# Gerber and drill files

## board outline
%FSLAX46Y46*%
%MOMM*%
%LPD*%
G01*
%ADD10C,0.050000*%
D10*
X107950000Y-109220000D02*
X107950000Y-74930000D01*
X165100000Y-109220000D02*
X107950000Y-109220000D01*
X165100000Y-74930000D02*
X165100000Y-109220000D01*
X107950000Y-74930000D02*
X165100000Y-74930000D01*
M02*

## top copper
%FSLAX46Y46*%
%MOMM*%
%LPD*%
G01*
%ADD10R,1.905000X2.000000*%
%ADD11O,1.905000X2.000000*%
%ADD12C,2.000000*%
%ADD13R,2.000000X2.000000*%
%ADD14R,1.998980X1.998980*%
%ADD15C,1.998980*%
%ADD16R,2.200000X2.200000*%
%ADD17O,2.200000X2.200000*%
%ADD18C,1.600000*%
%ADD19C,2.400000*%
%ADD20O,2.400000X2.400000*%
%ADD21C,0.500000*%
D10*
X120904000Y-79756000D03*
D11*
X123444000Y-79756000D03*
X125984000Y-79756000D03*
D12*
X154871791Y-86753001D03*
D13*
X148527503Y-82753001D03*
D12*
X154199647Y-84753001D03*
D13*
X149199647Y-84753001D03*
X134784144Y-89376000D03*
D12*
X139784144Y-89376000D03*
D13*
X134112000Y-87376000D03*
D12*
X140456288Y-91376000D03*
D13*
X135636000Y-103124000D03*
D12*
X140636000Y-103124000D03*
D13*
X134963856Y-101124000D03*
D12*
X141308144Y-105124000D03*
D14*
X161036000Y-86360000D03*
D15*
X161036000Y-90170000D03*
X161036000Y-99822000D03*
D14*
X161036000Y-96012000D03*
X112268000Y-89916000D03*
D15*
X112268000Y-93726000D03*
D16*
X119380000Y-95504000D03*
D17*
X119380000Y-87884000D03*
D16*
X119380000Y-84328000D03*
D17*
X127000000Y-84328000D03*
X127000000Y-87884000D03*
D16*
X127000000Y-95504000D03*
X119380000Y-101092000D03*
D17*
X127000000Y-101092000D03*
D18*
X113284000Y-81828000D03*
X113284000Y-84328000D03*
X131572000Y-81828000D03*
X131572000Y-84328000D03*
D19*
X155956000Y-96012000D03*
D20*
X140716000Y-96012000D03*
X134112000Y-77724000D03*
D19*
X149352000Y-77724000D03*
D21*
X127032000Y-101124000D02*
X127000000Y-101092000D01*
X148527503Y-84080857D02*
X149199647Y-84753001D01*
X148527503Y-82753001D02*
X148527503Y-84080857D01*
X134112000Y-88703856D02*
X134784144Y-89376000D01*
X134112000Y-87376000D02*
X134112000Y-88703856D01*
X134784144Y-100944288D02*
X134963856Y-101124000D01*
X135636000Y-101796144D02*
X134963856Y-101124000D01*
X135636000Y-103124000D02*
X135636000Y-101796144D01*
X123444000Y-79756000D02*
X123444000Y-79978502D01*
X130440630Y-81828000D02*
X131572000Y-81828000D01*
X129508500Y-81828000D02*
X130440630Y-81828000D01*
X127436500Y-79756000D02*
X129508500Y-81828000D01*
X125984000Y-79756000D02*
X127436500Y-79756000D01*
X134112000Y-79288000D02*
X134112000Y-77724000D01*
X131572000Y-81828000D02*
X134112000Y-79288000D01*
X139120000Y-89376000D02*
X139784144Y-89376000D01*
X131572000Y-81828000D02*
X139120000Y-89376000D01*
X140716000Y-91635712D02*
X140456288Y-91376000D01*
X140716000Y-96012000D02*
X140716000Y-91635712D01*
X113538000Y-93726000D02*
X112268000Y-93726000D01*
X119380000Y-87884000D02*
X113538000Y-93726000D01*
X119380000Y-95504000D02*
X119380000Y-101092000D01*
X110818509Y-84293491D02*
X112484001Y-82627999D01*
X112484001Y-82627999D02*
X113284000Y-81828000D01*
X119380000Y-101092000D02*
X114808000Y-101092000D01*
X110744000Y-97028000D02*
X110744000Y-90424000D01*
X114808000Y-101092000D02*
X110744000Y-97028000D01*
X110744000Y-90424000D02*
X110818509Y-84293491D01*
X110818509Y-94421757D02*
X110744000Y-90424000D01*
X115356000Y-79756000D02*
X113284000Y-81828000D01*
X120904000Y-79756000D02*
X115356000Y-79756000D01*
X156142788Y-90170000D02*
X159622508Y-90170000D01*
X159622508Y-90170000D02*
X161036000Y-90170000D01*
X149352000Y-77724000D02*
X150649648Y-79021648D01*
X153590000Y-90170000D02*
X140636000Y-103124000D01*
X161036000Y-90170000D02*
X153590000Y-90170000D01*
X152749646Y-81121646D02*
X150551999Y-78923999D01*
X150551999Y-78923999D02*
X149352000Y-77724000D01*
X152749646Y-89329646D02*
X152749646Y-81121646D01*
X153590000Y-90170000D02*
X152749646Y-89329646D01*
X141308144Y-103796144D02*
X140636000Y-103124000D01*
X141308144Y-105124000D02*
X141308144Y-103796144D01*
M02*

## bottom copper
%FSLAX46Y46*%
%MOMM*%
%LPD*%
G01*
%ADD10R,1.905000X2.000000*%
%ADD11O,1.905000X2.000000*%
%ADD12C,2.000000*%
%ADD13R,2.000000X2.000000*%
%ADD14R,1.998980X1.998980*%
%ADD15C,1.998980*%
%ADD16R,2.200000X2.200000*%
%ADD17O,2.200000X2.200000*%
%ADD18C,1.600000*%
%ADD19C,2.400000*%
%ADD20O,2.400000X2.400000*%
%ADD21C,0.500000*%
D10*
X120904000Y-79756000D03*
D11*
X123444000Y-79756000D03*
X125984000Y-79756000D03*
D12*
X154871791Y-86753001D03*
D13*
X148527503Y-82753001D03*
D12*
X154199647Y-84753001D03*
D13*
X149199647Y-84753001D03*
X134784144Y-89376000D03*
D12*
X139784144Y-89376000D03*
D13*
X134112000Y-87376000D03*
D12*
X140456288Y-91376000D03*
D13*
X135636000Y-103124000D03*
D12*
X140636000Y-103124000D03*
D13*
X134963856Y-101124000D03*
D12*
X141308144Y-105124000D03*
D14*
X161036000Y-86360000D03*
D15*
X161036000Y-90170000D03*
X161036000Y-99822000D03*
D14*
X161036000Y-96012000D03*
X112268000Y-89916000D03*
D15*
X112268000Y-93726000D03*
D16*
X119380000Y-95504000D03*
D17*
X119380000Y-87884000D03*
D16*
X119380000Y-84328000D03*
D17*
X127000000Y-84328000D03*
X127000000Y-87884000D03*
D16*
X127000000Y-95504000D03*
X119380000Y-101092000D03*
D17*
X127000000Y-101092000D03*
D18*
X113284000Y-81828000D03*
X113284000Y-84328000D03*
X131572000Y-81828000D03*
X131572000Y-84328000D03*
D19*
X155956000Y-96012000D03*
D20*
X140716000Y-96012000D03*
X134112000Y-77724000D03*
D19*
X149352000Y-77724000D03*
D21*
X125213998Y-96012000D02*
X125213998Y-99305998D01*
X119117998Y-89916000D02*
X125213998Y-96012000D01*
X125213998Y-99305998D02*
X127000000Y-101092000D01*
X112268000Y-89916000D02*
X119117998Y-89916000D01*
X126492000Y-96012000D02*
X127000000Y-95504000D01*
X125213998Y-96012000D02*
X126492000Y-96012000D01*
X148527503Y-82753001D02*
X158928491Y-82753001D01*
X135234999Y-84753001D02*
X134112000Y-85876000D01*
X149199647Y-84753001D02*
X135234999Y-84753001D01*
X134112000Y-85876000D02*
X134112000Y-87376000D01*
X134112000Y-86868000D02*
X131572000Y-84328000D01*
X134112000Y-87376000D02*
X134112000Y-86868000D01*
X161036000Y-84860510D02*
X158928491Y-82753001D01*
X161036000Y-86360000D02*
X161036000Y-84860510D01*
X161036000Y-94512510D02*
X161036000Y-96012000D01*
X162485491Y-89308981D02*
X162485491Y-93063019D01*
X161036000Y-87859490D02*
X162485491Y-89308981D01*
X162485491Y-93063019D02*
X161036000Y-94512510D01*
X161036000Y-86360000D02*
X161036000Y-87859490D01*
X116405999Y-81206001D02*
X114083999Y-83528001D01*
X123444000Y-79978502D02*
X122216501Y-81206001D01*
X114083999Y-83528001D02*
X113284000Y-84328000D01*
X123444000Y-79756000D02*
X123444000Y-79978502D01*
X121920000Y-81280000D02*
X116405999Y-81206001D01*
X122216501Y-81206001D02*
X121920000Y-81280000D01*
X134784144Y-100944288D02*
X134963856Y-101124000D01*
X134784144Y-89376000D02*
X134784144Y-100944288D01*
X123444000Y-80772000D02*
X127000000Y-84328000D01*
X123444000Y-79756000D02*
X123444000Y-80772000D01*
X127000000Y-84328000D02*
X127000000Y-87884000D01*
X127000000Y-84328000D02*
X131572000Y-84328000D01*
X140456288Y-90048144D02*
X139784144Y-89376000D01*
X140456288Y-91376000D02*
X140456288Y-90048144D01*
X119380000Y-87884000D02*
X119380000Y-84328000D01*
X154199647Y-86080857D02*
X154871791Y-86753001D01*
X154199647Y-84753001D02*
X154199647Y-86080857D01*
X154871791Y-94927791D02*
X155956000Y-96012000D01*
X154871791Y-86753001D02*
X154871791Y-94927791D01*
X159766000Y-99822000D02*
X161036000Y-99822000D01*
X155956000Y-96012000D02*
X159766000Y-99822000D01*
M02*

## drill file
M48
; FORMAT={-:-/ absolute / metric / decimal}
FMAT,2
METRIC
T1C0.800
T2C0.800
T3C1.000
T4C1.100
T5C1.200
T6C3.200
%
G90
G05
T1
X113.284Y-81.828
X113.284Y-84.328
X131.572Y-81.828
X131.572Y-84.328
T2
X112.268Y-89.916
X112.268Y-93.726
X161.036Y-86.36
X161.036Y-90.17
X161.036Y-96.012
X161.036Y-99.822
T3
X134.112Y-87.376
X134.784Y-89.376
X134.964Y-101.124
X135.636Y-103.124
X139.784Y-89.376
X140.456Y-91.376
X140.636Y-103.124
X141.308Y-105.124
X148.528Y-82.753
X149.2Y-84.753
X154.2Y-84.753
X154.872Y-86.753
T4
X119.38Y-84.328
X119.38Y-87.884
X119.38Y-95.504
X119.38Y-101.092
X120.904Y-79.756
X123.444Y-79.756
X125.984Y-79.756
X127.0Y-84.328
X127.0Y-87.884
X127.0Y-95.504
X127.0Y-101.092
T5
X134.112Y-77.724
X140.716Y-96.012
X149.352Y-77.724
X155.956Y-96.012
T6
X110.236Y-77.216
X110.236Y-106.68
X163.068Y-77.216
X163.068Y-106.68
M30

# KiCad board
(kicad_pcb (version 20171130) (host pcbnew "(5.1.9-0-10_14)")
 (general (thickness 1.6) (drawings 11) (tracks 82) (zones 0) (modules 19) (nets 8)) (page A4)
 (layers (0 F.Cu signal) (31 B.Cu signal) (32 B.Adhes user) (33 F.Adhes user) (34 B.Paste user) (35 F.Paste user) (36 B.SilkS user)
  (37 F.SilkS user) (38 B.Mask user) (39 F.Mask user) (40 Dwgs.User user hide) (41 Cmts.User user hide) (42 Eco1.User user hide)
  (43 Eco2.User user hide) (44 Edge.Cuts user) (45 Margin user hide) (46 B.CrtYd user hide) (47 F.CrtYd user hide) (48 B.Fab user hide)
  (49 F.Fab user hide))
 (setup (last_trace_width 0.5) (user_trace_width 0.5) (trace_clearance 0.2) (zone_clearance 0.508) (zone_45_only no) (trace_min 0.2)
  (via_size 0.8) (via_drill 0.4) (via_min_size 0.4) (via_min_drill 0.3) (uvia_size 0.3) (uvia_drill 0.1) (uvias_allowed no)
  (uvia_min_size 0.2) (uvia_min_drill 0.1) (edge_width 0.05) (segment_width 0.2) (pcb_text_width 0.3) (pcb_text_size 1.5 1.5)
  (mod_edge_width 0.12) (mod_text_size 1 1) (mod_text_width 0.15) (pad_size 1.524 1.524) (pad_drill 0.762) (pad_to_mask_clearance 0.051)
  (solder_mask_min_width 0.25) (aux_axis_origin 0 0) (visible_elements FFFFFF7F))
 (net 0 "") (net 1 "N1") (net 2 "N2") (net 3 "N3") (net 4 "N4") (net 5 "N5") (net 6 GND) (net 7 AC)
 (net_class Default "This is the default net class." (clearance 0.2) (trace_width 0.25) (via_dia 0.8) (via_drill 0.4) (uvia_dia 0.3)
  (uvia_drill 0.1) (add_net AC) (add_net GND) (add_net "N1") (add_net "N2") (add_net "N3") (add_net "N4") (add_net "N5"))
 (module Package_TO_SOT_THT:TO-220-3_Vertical (layer F.Cu) (at 120.904 79.756)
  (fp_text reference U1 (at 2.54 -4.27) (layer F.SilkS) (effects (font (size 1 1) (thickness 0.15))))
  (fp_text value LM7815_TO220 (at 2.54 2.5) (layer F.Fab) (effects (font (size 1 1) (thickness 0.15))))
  (pad 1 thru_hole rect (at 0 0) (size 1.905 2) (drill 1.1) (layers *.Cu *.Mask) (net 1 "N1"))
  (pad 2 thru_hole oval (at 2.54 0) (size 1.905 2) (drill 1.1) (layers *.Cu *.Mask) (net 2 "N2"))
  (pad 3 thru_hole oval (at 5.08 0) (size 1.905 2) (drill 1.1) (layers *.Cu *.Mask) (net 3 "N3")))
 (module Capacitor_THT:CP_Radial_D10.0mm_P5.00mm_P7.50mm (layer F.Cu) (at 149.199647 84.753001)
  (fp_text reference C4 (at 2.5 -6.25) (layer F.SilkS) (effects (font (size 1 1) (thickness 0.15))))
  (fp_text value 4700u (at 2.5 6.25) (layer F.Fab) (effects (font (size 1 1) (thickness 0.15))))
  (pad 2 thru_hole circle (at 5.672144 2) (size 2 2) (drill 1) (layers *.Cu *.Mask) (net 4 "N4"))
  (pad 1 thru_hole rect (at -0.672144 -2) (size 2 2) (drill 1) (layers *.Cu *.Mask) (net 2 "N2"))
  (pad 2 thru_hole circle (at 5 0) (size 2 2) (drill 1) (layers *.Cu *.Mask) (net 4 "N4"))
  (pad 1 thru_hole rect (at 0 0) (size 2 2) (drill 1) (layers *.Cu *.Mask) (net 2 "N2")))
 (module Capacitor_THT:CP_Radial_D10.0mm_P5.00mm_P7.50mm (layer F.Cu) (at 134.784144 89.376)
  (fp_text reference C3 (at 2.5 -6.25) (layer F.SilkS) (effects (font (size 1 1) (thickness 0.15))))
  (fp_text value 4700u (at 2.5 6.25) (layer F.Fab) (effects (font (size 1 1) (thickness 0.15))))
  (pad 1 thru_hole rect (at 0 0) (size 2 2) (drill 1) (layers *.Cu *.Mask) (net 2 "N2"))
  (pad 2 thru_hole circle (at 5 0) (size 2 2) (drill 1) (layers *.Cu *.Mask) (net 3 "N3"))
  (pad 1 thru_hole rect (at -0.672144 -2) (size 2 2) (drill 1) (layers *.Cu *.Mask) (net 2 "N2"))
  (pad 2 thru_hole circle (at 5.672144 2) (size 2 2) (drill 1) (layers *.Cu *.Mask) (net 3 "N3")))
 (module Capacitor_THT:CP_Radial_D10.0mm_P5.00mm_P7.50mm (layer F.Cu) (at 135.636 103.124)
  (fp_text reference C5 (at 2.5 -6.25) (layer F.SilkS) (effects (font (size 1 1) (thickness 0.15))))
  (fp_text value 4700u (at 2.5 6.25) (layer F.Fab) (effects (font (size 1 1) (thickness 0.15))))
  (pad 1 thru_hole rect (at 0 0) (size 2 2) (drill 1) (layers *.Cu *.Mask) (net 2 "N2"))
  (pad 2 thru_hole circle (at 5 0) (size 2 2) (drill 1) (layers *.Cu *.Mask) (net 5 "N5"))
  (pad 1 thru_hole rect (at -0.672144 -2) (size 2 2) (drill 1) (layers *.Cu *.Mask) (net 2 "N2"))
  (pad 2 thru_hole circle (at 5.672144 2) (size 2 2) (drill 1) (layers *.Cu *.Mask) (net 5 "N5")))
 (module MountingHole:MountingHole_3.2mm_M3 (layer F.Cu) (at 110.236 77.216)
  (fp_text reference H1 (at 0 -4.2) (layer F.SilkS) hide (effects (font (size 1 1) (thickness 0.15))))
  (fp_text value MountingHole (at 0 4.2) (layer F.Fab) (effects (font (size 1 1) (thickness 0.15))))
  (pad 1 np_thru_hole circle (at 0 0) (size 3.2 3.2) (drill 3.2) (layers *.Cu *.Mask)))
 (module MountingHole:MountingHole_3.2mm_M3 (layer F.Cu) (at 110.236 106.68)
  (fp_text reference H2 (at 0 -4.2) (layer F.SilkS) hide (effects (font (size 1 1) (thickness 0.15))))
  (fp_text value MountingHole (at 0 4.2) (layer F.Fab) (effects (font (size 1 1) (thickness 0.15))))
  (pad 1 np_thru_hole circle (at 0 0) (size 3.2 3.2) (drill 3.2) (layers *.Cu *.Mask)))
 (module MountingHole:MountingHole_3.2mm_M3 (layer F.Cu) (at 163.068 77.216)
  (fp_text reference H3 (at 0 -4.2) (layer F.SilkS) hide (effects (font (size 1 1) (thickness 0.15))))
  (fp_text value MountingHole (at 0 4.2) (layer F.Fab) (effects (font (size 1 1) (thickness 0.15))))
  (pad 1 np_thru_hole circle (at 0 0) (size 3.2 3.2) (drill 3.2) (layers *.Cu *.Mask)))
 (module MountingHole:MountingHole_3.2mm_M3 (layer F.Cu) (at 163.068 106.68)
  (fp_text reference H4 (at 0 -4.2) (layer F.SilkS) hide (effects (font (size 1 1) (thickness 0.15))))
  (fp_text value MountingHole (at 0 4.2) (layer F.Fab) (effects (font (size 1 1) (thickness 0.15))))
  (pad 1 np_thru_hole circle (at 0 0) (size 3.2 3.2) (drill 3.2) (layers *.Cu *.Mask)))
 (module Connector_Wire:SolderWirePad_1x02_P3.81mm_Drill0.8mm (layer F.Cu) (at 161.036 86.36 270)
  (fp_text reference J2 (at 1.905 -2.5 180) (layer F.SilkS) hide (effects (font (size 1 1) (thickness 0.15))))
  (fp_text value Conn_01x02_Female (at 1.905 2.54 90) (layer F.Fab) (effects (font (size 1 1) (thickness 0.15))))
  (pad 1 thru_hole rect (at 0 0 270) (size 1.99898 1.99898) (drill 0.8001) (layers *.Cu *.Mask) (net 2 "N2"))
  (pad 2 thru_hole circle (at 3.81 0 270) (size 1.99898 1.99898) (drill 0.8001) (layers *.Cu *.Mask) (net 5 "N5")))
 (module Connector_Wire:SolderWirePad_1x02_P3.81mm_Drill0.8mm (layer F.Cu) (at 161.036 96.012 270)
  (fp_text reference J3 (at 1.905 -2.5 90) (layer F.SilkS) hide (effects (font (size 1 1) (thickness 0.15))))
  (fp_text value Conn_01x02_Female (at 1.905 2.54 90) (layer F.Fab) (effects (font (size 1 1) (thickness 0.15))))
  (pad 2 thru_hole circle (at 3.81 0 270) (size 1.99898 1.99898) (drill 0.8001) (layers *.Cu *.Mask) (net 4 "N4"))
  (pad 1 thru_hole rect (at 0 0 270) (size 1.99898 1.99898) (drill 0.8001) (layers *.Cu *.Mask) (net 2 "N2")))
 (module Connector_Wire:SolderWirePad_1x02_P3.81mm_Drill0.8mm (layer F.Cu) (at 112.268 89.916 270)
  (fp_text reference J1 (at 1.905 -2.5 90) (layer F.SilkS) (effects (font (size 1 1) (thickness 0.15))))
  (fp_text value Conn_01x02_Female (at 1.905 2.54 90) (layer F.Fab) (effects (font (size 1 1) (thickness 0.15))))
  (pad 1 thru_hole rect (at 0 0 270) (size 1.99898 1.99898) (drill 0.8001) (layers *.Cu *.Mask) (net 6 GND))
  (pad 2 thru_hole circle (at 3.81 0 270) (size 1.99898 1.99898) (drill 0.8001) (layers *.Cu *.Mask) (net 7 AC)))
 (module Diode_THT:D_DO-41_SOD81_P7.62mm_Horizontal (layer F.Cu) (at 119.38 95.504 90)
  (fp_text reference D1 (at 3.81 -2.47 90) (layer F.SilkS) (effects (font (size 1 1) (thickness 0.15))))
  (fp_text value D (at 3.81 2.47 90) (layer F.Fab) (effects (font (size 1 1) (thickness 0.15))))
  (pad 1 thru_hole rect (at 0 0 90) (size 2.2 2.2) (drill 1.1) (layers *.Cu *.Mask) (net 1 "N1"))
  (pad 2 thru_hole oval (at 7.62 0 90) (size 2.2 2.2) (drill 1.1) (layers *.Cu *.Mask) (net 7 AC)))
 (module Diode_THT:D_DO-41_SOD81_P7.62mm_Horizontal (layer F.Cu) (at 119.38 84.328)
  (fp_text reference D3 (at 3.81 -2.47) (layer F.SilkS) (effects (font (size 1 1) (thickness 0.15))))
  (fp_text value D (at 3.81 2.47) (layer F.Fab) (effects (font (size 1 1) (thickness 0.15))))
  (pad 1 thru_hole rect (at 0 0) (size 2.2 2.2) (drill 1.1) (layers *.Cu *.Mask) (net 7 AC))
  (pad 2 thru_hole oval (at 7.62 0) (size 2.2 2.2) (drill 1.1) (layers *.Cu *.Mask) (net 2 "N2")))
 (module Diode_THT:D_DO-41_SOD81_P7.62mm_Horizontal (layer F.Cu) (at 127 95.504 90)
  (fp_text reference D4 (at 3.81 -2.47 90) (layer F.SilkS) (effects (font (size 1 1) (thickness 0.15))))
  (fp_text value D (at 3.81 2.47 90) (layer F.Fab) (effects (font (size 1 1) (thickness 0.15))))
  (pad 2 thru_hole oval (at 7.62 0 90) (size 2.2 2.2) (drill 1.1) (layers *.Cu *.Mask) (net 2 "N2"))
  (pad 1 thru_hole rect (at 0 0 90) (size 2.2 2.2) (drill 1.1) (layers *.Cu *.Mask) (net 6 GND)))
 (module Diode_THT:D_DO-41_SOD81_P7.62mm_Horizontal (layer F.Cu) (at 119.38 101.092)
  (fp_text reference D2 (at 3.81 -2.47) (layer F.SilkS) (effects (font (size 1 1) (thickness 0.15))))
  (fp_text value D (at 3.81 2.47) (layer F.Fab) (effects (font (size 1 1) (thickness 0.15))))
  (pad 1 thru_hole rect (at 0 0) (size 2.2 2.2) (drill 1.1) (layers *.Cu *.Mask) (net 1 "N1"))
  (pad 2 thru_hole oval (at 7.62 0) (size 2.2 2.2) (drill 1.1) (layers *.Cu *.Mask) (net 6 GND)))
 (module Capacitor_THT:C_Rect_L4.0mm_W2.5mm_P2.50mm (layer F.Cu) (at 113.284 81.828 270)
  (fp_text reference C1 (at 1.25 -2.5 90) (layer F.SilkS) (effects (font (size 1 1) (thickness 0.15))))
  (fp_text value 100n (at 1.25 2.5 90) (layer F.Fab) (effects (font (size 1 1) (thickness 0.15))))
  (pad 1 thru_hole circle (at 0 0 270) (size 1.6 1.6) (drill 0.8) (layers *.Cu *.Mask) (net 1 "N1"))
  (pad 2 thru_hole circle (at 2.5 0 270) (size 1.6 1.6) (drill 0.8) (layers *.Cu *.Mask) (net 2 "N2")))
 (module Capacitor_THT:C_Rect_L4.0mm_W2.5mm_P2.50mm (layer F.Cu) (at 131.572 84.328 90)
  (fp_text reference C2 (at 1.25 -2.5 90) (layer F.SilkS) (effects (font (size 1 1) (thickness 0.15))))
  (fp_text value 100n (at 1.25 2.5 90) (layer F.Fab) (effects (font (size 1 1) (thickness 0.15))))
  (pad 2 thru_hole circle (at 2.5 0 90) (size 1.6 1.6) (drill 0.8) (layers *.Cu *.Mask) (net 3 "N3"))
  (pad 1 thru_hole circle (at 0 0 90) (size 1.6 1.6) (drill 0.8) (layers *.Cu *.Mask) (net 2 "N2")))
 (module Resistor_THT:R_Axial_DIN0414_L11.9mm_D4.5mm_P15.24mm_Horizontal (layer F.Cu) (at 155.956 96.012 180)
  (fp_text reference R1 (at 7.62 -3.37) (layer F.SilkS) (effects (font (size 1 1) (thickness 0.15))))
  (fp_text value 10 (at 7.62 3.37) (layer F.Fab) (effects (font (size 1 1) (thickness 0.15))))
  (pad 1 thru_hole circle (at 0 0 180) (size 2.4 2.4) (drill 1.2) (layers *.Cu *.Mask) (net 4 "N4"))
  (pad 2 thru_hole oval (at 15.24 0 180) (size 2.4 2.4) (drill 1.2) (layers *.Cu *.Mask) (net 3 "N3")))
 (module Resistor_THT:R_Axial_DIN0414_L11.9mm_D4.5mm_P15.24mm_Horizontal (layer F.Cu) (at 149.352 77.724 180)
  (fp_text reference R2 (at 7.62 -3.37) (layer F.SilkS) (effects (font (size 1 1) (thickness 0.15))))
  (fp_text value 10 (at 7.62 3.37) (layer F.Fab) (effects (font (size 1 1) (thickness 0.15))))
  (pad 2 thru_hole oval (at 15.24 0 180) (size 2.4 2.4) (drill 1.2) (layers *.Cu *.Mask) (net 3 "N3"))
  (pad 1 thru_hole circle (at 0 0 180) (size 2.4 2.4) (drill 1.2) (layers *.Cu *.Mask) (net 5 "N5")))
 (gr_line (start 107.95 109.22) (end 107.95 74.93) (layer Edge.Cuts) (width 0.05))
 (gr_line (start 165.1 109.22) (end 107.95 109.22) (layer Edge.Cuts) (width 0.05))
 (gr_line (start 165.1 74.93) (end 165.1 109.22) (layer Edge.Cuts) (width 0.05))
 (gr_line (start 107.95 74.93) (end 165.1 74.93) (layer Edge.Cuts) (width 0.05))
 (segment (start 127.032 101.124) (end 127 101.092) (width 0.5) (layer F.Cu) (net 6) (status 30))
 (segment (start 125.213998 96.012) (end 125.213998 99.305998) (width 0.5) (layer B.Cu) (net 6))
 (segment (start 119.117998 89.916) (end 125.213998 96.012) (width 0.5) (layer B.Cu) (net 6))
 (segment (start 125.213998 99.305998) (end 127 101.092) (width 0.5) (layer B.Cu) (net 6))
 (segment (start 112.268 89.916) (end 119.117998 89.916) (width 0.5) (layer B.Cu) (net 6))
 (segment (start 126.492 96.012) (end 127 95.504) (width 0.5) (layer B.Cu) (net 6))
 (segment (start 125.213998 96.012) (end 126.492 96.012) (width 0.5) (layer B.Cu) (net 6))
 (segment (start 148.527503 84.080857) (end 149.199647 84.753001) (width 0.5) (layer F.Cu) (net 2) (status 30))
 (segment (start 148.527503 82.753001) (end 148.527503 84.080857) (width 0.5) (layer F.Cu) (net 2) (status 30))
 (segment (start 148.527503 82.753001) (end 158.928491 82.753001) (width 0.5) (layer B.Cu) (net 2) (status 10))
 (segment (start 135.234999 84.753001) (end 134.112 85.876) (width 0.5) (layer B.Cu) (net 2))
 (segment (start 149.199647 84.753001) (end 135.234999 84.753001) (width 0.5) (layer B.Cu) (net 2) (status 10))
 (segment (start 134.112 85.876) (end 134.112 87.376) (width 0.5) (layer B.Cu) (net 2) (status 20))
 (segment (start 134.112 86.868) (end 131.572 84.328) (width 0.5) (layer B.Cu) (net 2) (status 30))
 (segment (start 134.112 87.376) (end 134.112 86.868) (width 0.5) (layer B.Cu) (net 2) (status 30))
 (segment (start 134.112 88.703856) (end 134.784144 89.376) (width 0.5) (layer F.Cu) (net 2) (status 30))
 (segment (start 134.112 87.376) (end 134.112 88.703856) (width 0.5) (layer F.Cu) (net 2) (status 30))
 (segment (start 134.784144 100.944288) (end 134.963856 101.124) (width 0.5) (layer F.Cu) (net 2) (status 30))
 (segment (start 135.636 101.796144) (end 134.963856 101.124) (width 0.5) (layer F.Cu) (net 2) (status 30))
 (segment (start 135.636 103.124) (end 135.636 101.796144) (width 0.5) (layer F.Cu) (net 2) (status 30))
 (segment (start 123.444 79.756) (end 123.444 79.978502) (width 0.5) (layer F.Cu) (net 2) (status 30))
 (segment (start 161.036 84.86051) (end 158.928491 82.753001) (width 0.5) (layer B.Cu) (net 2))
 (segment (start 161.036 86.36) (end 161.036 84.86051) (width 0.5) (layer B.Cu) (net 2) (status 10))
 (segment (start 161.036 94.51251) (end 161.036 96.012) (width 0.5) (layer B.Cu) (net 2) (status 20))
 (segment (start 162.485491 89.308981) (end 162.485491 93.063019) (width 0.5) (layer B.Cu) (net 2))
 (segment (start 161.036 87.85949) (end 162.485491 89.308981) (width 0.5) (layer B.Cu) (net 2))
 (segment (start 162.485491 93.063019) (end 161.036 94.51251) (width 0.5) (layer B.Cu) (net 2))
 (segment (start 161.036 86.36) (end 161.036 87.85949) (width 0.5) (layer B.Cu) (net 2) (status 10))
 (segment (start 116.405999 81.206001) (end 114.083999 83.528001) (width 0.5) (layer B.Cu) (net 2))
 (segment (start 123.444 79.978502) (end 122.216501 81.206001) (width 0.5) (layer B.Cu) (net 2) (status 10))
 (segment (start 114.083999 83.528001) (end 113.284 84.328) (width 0.5) (layer B.Cu) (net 2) (status 20))
 (segment (start 123.444 79.756) (end 123.444 79.978502) (width 0.5) (layer B.Cu) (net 2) (status 30))
 (segment (start 121.92 81.28) (end 116.405999 81.206001) (width 0.5) (layer B.Cu) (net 2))
 (segment (start 122.216501 81.206001) (end 121.92 81.28) (width 0.5) (layer B.Cu) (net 2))
 (segment (start 134.784144 100.944288) (end 134.963856 101.124) (width 0.5) (layer B.Cu) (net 2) (status 30))
 (segment (start 134.784144 89.376) (end 134.784144 100.944288) (width 0.5) (layer B.Cu) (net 2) (status 30))
 (segment (start 123.444 80.772) (end 127 84.328) (width 0.5) (layer B.Cu) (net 2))
 (segment (start 123.444 79.756) (end 123.444 80.772) (width 0.5) (layer B.Cu) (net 2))
 (segment (start 127 84.328) (end 127 87.884) (width 0.5) (layer B.Cu) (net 2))
 (segment (start 127 84.328) (end 131.572 84.328) (width 0.5) (layer B.Cu) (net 2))
 (segment (start 140.456288 90.048144) (end 139.784144 89.376) (width 0.5) (layer B.Cu) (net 3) (status 30))
 (segment (start 140.456288 91.376) (end 140.456288 90.048144) (width 0.5) (layer B.Cu) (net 3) (status 30))
 (segment (start 130.44063 81.828) (end 131.572 81.828) (width 0.5) (layer F.Cu) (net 3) (status 20))
 (segment (start 129.5085 81.828) (end 130.44063 81.828) (width 0.5) (layer F.Cu) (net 3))
 (segment (start 127.4365 79.756) (end 129.5085 81.828) (width 0.5) (layer F.Cu) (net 3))
 (segment (start 125.984 79.756) (end 127.4365 79.756) (width 0.5) (layer F.Cu) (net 3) (status 10))
 (segment (start 134.112 79.288) (end 134.112 77.724) (width 0.5) (layer F.Cu) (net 3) (status 20))
 (segment (start 131.572 81.828) (end 134.112 79.288) (width 0.5) (layer F.Cu) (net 3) (status 10))
 (segment (start 139.12 89.376) (end 139.784144 89.376) (width 0.5) (layer F.Cu) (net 3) (status 30))
 (segment (start 131.572 81.828) (end 139.12 89.376) (width 0.5) (layer F.Cu) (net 3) (status 30))
 (segment (start 140.716 91.635712) (end 140.456288 91.376) (width 0.5) (layer F.Cu) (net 3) (status 30))
 (segment (start 140.716 96.012) (end 140.716 91.635712) (width 0.5) (layer F.Cu) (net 3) (status 30))
 (segment (start 113.538 93.726) (end 112.268 93.726) (width 0.5) (layer F.Cu) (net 7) (status 20))
 (segment (start 119.38 87.884) (end 113.538 93.726) (width 0.5) (layer F.Cu) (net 7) (status 10))
 (segment (start 119.38 87.884) (end 119.38 84.328) (width 0.5) (layer B.Cu) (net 7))
 (segment (start 119.38 95.504) (end 119.38 101.092) (width 0.5) (layer F.Cu) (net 1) (status 30))
 (segment (start 110.818509 84.293491) (end 112.484001 82.627999) (width 0.5) (layer F.Cu) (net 1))
 (segment (start 112.484001 82.627999) (end 113.284 81.828) (width 0.5) (layer F.Cu) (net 1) (status 20))
 (segment (start 119.38 101.092) (end 114.808 101.092) (width 0.5) (layer F.Cu) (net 1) (status 10))
 (segment (start 110.744 97.028) (end 110.744 90.424) (width 0.5) (layer F.Cu) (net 1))
 (segment (start 114.808 101.092) (end 110.744 97.028) (width 0.5) (layer F.Cu) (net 1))
 (segment (start 110.744 90.424) (end 110.818509 84.293491) (width 0.5) (layer F.Cu) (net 1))
 (segment (start 110.818509 94.421757) (end 110.744 90.424) (width 0.5) (layer F.Cu) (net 1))
 (segment (start 115.356 79.756) (end 113.284 81.828) (width 0.5) (layer F.Cu) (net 1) (status 20))
 (segment (start 120.904 79.756) (end 115.356 79.756) (width 0.5) (layer F.Cu) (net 1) (status 10))
 (segment (start 154.199647 86.080857) (end 154.871791 86.753001) (width 0.5) (layer B.Cu) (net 4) (status 30))
 (segment (start 154.199647 84.753001) (end 154.199647 86.080857) (width 0.5) (layer B.Cu) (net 4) (status 30))
 (segment (start 154.871791 94.927791) (end 155.956 96.012) (width 0.5) (layer B.Cu) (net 4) (status 20))
 (segment (start 154.871791 86.753001) (end 154.871791 94.927791) (width 0.5) (layer B.Cu) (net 4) (status 10))
 (segment (start 159.766 99.822) (end 161.036 99.822) (width 0.5) (layer B.Cu) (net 4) (status 20))
 (segment (start 155.956 96.012) (end 159.766 99.822) (width 0.5) (layer B.Cu) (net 4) (status 10))
 (segment (start 156.142788 90.17) (end 159.622508 90.17) (width 0.5) (layer F.Cu) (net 5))
 (segment (start 159.622508 90.17) (end 161.036 90.17) (width 0.5) (layer F.Cu) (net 5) (status 20))
 (segment (start 149.352 77.724) (end 150.649648 79.021648) (width 0.5) (layer F.Cu) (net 5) (status 10))
 (segment (start 153.59 90.17) (end 140.636 103.124) (width 0.5) (layer F.Cu) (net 5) (status 20))
 (segment (start 161.036 90.17) (end 153.59 90.17) (width 0.5) (layer F.Cu) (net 5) (status 10))
 (segment (start 152.749646 81.121646) (end 150.551999 78.923999) (width 0.5) (layer F.Cu) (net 5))
 (segment (start 150.551999 78.923999) (end 149.352 77.724) (width 0.5) (layer F.Cu) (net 5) (status 20))
 (segment (start 152.749646 89.329646) (end 152.749646 81.121646) (width 0.5) (layer F.Cu) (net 5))
 (segment (start 153.59 90.17) (end 152.749646 89.329646) (width 0.5) (layer F.Cu) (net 5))
 (segment (start 141.308144 103.796144) (end 140.636 103.124) (width 0.5) (layer F.Cu) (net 5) (status 30))
 (segment (start 141.308144 105.124) (end 141.308144 103.796144) (width 0.5) (layer F.Cu) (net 5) (status 30)))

